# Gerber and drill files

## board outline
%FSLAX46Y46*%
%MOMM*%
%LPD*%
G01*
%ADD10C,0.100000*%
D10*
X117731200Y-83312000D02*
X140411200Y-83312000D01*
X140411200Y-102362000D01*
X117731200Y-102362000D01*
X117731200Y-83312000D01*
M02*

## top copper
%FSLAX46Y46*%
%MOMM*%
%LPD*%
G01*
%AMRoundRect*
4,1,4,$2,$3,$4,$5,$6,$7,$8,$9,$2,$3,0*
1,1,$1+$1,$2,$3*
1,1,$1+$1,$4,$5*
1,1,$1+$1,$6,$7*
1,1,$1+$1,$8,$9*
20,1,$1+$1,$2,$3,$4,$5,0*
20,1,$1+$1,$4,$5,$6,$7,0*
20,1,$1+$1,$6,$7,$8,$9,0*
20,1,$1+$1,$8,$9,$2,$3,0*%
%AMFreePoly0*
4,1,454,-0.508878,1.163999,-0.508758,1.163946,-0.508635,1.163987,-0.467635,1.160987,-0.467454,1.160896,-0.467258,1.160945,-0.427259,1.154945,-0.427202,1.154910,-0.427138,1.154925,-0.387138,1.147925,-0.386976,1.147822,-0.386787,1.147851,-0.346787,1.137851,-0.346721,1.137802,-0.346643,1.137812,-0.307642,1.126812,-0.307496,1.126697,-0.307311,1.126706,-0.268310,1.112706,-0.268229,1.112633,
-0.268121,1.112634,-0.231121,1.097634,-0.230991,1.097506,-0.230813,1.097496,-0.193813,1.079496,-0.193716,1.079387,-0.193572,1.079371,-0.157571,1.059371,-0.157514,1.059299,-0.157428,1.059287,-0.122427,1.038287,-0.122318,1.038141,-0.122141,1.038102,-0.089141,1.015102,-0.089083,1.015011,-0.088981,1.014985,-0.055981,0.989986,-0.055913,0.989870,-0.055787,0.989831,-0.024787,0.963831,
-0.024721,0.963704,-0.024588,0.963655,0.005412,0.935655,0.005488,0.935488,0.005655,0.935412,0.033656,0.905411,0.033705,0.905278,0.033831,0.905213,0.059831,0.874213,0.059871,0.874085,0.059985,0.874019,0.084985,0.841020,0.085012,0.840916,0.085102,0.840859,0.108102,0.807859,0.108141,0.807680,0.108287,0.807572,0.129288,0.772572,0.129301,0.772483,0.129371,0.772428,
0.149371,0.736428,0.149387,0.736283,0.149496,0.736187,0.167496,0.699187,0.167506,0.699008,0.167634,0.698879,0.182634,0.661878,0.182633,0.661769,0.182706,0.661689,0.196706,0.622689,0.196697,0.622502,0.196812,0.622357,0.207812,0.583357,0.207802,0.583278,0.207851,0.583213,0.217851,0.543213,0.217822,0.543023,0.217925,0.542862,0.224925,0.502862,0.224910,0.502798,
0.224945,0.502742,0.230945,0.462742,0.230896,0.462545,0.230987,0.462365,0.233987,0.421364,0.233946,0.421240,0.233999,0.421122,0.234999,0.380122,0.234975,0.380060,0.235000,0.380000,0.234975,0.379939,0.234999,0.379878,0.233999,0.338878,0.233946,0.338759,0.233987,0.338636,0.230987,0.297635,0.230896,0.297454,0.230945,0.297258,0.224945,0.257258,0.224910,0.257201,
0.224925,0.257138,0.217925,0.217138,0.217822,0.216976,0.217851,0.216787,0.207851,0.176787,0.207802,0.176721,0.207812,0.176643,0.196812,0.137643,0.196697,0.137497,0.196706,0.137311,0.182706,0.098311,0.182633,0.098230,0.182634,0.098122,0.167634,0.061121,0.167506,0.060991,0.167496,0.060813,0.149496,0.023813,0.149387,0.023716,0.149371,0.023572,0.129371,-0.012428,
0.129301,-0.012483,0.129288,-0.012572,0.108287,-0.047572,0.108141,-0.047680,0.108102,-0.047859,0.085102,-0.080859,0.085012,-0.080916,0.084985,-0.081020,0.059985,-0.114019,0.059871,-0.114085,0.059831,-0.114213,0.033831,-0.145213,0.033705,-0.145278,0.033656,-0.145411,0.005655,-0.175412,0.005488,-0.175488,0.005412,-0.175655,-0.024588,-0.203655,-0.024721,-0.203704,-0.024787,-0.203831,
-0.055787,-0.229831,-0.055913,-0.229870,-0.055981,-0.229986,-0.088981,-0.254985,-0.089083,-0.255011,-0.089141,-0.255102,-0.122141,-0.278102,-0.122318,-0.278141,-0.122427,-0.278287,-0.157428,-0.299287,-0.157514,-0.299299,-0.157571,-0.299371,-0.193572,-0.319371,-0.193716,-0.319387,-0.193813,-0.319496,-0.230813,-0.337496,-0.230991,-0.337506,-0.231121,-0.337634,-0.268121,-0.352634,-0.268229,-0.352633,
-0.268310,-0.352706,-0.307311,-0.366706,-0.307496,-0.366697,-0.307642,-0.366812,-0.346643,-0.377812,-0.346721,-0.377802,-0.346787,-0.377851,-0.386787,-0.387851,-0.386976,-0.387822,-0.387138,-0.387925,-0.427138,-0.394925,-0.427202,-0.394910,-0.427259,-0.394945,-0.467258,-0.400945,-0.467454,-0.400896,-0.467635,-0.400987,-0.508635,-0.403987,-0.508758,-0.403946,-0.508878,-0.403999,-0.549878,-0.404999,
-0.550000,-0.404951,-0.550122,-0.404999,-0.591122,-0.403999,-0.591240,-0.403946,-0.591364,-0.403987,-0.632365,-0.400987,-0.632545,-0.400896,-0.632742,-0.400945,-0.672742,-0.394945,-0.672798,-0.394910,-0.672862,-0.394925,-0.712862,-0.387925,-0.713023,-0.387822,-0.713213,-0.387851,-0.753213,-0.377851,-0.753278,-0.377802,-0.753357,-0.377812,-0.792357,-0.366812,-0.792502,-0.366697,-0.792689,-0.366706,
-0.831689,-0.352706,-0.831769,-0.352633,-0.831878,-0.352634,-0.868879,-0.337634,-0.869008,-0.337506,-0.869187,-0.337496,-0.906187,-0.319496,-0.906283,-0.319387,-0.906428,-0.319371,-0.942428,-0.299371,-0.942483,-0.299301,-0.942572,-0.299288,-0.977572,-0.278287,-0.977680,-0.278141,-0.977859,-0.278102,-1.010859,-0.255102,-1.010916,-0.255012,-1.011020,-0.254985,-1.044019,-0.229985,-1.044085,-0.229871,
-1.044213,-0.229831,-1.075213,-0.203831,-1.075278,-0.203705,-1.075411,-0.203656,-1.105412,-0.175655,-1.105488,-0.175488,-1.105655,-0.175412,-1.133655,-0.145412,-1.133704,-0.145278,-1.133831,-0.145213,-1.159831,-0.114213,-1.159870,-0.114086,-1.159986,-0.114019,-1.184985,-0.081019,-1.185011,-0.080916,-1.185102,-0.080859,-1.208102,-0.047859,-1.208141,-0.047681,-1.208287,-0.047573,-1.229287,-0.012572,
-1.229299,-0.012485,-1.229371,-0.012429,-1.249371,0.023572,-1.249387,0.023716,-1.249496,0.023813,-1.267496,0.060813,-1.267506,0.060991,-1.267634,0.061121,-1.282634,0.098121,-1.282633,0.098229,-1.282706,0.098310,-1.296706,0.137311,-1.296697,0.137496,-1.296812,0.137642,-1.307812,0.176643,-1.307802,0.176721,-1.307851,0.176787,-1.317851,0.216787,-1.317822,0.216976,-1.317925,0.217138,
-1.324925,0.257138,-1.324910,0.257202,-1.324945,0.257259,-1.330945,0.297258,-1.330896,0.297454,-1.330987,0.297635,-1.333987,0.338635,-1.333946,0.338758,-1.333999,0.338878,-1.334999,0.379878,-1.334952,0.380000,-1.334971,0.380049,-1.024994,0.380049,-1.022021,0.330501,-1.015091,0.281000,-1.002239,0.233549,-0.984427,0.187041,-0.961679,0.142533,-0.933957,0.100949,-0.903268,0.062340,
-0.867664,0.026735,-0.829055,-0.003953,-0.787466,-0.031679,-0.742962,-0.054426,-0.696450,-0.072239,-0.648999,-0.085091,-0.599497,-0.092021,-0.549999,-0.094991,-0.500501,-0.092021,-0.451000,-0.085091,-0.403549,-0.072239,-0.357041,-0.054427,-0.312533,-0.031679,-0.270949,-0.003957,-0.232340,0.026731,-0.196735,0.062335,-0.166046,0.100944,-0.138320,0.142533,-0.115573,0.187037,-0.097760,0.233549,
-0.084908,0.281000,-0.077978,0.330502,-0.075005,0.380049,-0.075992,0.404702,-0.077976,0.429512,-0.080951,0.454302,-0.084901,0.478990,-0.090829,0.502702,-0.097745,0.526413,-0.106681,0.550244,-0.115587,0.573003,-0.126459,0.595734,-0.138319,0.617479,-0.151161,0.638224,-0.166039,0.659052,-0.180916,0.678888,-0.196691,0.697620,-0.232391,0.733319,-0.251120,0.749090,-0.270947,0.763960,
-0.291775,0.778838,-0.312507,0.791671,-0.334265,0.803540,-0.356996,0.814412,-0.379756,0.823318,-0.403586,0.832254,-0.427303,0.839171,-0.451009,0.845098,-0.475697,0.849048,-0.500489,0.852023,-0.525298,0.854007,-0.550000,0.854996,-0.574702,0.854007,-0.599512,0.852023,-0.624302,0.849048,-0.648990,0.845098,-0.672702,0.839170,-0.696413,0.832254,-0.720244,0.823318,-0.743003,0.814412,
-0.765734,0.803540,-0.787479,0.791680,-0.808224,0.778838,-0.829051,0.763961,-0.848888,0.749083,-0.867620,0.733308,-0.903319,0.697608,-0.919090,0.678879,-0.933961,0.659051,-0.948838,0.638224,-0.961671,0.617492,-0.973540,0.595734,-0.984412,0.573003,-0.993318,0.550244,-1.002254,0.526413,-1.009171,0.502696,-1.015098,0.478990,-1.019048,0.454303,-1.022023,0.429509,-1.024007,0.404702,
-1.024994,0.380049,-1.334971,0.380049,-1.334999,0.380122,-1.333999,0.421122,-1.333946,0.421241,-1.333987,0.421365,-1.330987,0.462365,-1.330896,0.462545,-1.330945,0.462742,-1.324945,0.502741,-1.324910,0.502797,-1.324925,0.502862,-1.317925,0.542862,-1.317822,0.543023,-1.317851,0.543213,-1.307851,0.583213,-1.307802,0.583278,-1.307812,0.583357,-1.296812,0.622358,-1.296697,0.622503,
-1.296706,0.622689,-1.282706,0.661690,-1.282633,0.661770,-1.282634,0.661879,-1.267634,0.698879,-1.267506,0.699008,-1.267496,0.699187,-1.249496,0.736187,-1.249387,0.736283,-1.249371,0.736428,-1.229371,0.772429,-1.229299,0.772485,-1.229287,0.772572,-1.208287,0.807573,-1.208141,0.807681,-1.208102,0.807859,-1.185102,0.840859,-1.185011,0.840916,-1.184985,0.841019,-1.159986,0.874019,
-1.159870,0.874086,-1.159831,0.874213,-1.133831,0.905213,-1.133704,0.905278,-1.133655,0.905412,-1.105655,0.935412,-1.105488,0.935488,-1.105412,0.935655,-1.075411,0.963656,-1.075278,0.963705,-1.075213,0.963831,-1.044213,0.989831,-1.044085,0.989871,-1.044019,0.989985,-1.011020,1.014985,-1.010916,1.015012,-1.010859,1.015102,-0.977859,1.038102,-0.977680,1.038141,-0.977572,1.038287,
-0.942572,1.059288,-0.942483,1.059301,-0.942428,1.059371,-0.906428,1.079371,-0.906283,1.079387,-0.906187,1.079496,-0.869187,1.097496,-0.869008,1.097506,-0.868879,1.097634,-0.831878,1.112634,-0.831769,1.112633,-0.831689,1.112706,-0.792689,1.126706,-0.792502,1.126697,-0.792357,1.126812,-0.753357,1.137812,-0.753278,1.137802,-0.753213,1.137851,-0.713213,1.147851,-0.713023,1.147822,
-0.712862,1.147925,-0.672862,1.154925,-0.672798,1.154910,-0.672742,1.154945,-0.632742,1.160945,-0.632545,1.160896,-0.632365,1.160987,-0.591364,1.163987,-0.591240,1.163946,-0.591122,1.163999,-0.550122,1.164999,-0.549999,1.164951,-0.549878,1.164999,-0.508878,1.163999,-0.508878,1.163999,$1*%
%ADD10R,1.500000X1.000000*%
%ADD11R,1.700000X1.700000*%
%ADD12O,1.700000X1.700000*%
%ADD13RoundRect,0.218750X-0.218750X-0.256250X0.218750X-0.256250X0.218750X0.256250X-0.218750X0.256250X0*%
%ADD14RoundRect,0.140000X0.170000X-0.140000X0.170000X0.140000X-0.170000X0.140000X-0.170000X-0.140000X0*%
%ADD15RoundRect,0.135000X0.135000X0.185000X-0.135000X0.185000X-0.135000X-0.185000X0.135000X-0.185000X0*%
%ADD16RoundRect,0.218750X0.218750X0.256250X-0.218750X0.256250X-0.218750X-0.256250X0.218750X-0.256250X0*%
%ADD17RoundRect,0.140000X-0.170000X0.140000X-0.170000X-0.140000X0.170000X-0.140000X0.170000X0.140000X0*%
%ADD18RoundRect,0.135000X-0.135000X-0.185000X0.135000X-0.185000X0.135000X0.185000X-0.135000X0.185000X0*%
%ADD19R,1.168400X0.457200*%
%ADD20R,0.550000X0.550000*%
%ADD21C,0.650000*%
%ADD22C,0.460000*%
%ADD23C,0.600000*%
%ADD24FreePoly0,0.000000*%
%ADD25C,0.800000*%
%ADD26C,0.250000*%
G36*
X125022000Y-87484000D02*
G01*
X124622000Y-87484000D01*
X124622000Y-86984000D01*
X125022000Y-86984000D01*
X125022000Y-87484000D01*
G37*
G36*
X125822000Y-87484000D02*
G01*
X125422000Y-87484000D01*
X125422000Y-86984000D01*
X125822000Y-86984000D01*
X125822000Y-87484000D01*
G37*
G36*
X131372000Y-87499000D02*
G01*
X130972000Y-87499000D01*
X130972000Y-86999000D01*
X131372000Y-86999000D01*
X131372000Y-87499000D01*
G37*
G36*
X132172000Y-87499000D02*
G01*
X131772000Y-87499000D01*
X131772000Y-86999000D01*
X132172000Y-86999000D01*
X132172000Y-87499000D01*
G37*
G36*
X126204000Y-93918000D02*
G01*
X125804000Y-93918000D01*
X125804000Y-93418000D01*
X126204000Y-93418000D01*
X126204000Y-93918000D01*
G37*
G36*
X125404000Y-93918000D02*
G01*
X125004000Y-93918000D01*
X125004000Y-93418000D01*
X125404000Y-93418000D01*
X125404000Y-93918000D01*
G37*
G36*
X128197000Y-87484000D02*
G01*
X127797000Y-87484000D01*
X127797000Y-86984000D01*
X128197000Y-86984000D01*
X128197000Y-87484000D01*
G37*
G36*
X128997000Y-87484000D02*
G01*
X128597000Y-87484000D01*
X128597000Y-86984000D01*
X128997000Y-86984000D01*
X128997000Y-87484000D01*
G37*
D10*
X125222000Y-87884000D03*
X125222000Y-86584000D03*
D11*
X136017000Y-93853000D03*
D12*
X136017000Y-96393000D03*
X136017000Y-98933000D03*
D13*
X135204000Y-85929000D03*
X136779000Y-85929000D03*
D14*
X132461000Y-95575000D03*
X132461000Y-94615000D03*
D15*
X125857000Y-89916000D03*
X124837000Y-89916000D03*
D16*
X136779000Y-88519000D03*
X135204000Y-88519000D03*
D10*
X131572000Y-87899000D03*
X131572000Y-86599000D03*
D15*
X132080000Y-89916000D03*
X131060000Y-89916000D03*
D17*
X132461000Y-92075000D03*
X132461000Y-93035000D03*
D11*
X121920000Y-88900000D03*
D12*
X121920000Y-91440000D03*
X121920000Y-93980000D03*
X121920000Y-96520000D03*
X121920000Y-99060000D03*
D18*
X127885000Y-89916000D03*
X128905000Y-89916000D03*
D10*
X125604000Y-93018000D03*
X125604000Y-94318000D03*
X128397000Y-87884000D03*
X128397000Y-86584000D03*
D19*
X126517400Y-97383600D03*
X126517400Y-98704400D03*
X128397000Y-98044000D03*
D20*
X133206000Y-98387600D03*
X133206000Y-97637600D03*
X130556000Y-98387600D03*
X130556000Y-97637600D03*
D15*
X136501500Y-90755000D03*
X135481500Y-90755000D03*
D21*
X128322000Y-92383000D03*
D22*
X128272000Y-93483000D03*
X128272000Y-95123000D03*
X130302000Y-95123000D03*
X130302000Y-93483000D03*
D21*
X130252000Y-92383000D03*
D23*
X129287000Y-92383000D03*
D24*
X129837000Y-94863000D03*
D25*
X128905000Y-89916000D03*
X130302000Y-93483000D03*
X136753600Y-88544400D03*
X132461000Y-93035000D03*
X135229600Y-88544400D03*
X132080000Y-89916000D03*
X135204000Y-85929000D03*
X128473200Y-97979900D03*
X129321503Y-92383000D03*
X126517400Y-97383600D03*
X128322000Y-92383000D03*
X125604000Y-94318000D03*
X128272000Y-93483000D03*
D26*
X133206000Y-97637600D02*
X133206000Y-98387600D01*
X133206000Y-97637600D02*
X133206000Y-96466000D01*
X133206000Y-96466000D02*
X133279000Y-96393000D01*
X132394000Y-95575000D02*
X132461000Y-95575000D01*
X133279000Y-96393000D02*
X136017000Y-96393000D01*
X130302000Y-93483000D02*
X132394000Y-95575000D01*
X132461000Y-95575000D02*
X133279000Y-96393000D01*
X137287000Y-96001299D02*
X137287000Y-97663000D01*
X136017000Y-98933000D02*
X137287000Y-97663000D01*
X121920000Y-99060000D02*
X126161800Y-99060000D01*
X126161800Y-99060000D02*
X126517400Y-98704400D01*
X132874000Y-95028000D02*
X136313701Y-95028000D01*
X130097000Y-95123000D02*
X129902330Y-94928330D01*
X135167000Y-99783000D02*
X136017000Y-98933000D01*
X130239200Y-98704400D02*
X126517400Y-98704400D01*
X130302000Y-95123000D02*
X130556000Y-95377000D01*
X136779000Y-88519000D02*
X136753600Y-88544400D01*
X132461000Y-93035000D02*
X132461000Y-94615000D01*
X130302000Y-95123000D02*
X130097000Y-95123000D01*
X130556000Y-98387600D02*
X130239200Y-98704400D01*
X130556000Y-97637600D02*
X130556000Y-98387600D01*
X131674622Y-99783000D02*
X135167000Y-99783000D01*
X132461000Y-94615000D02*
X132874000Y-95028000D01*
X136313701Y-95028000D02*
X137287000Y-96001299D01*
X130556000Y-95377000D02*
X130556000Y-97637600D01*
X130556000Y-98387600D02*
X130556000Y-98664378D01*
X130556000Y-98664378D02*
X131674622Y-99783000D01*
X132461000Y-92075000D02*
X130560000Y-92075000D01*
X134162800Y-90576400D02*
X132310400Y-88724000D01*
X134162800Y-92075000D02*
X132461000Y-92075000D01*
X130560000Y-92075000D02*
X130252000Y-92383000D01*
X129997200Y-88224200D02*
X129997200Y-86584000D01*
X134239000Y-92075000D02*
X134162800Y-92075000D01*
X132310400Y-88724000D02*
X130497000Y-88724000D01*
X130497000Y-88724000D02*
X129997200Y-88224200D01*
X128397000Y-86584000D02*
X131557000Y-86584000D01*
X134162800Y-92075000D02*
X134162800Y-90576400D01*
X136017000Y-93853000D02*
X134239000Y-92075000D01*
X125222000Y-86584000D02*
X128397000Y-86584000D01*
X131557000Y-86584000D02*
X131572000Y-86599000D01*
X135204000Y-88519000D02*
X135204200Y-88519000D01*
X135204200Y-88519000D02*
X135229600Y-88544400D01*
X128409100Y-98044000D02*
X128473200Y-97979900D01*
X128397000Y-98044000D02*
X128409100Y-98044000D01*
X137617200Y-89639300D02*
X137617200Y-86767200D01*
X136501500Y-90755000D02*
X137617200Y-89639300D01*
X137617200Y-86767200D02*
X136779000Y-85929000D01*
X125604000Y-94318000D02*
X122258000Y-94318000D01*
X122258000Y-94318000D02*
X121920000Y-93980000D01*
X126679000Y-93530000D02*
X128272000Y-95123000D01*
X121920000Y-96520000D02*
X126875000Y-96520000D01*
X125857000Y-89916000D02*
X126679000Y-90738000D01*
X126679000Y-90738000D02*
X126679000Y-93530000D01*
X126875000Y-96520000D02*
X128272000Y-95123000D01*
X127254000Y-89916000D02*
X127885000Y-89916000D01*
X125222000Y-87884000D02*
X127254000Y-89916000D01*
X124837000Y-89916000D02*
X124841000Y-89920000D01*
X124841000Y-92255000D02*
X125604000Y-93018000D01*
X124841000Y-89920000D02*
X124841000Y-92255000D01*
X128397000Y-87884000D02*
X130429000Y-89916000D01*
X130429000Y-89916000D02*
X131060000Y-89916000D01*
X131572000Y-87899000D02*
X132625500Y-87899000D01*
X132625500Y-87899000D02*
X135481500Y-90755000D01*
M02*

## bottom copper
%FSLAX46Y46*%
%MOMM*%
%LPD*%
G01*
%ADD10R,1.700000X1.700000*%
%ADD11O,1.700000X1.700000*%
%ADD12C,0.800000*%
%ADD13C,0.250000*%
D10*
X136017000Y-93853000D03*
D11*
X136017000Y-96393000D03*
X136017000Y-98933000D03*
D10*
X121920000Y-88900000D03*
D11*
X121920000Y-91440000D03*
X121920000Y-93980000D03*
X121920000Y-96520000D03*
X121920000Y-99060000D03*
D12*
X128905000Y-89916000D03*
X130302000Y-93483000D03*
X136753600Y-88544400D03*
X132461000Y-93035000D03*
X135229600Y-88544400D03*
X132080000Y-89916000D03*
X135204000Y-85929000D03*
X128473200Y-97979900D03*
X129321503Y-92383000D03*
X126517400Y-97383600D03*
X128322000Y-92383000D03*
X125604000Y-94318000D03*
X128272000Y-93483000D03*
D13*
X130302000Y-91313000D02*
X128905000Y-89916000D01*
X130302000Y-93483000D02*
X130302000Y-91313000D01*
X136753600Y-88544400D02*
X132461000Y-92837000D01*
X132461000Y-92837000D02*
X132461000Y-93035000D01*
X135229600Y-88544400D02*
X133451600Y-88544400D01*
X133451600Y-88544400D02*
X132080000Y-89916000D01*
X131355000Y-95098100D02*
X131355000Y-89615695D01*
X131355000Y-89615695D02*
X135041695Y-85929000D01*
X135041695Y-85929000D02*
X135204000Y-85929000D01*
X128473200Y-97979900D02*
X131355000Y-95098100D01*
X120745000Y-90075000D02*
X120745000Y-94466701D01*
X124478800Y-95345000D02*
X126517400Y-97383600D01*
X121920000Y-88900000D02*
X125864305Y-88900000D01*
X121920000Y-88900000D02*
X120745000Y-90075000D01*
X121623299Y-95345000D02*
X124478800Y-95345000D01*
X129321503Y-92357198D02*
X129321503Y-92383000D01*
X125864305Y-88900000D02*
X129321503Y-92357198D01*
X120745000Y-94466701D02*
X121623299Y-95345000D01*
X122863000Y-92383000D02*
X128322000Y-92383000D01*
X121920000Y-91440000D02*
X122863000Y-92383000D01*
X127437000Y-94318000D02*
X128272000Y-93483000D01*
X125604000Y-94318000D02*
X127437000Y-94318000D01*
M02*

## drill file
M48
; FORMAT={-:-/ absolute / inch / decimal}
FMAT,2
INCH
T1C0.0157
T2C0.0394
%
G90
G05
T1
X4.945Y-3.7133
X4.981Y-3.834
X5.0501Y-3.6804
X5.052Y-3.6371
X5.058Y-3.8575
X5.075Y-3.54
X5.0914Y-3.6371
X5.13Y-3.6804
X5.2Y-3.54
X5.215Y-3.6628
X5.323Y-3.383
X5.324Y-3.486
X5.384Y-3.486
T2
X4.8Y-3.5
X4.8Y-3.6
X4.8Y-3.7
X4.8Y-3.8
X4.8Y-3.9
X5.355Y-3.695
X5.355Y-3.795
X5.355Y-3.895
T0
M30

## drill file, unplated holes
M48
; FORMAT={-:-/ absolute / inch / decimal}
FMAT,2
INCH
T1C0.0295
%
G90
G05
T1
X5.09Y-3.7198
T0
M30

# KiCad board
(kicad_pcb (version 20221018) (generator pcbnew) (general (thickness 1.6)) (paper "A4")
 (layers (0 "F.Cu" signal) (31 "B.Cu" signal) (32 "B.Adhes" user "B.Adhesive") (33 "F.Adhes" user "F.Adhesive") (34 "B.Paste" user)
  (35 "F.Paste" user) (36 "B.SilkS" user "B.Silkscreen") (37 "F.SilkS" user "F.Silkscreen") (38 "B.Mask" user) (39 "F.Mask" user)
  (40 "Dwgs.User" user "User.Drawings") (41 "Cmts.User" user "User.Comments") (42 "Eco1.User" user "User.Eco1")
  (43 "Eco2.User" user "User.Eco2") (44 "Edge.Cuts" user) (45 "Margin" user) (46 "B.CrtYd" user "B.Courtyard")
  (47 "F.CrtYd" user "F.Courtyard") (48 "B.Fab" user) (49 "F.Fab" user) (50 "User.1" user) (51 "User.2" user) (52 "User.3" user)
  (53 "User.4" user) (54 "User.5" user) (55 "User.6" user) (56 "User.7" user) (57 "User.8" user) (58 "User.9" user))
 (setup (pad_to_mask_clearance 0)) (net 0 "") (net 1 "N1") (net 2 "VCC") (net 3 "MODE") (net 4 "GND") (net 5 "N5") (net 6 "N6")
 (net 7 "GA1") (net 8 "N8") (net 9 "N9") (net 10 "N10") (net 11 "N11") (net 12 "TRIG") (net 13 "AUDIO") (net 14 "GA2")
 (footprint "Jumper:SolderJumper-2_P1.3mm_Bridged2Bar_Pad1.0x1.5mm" (layer "F.Cu") (at 125.222 87.234 90) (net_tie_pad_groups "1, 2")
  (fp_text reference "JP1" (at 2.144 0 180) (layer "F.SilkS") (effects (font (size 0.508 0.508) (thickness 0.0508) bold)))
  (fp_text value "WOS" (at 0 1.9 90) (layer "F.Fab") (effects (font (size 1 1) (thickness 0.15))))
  (fp_poly (pts (xy -0.25 -0.6) (xy 0.25 -0.6) (xy 0.25 -0.2) (xy -0.25 -0.2)) (stroke (width 0) (type solid)) (fill solid) (layer "F.Cu"))
  (fp_poly (pts (xy -0.25 0.2) (xy 0.25 0.2) (xy 0.25 0.6) (xy -0.25 0.6)) (stroke (width 0) (type solid)) (fill solid) (layer "F.Cu"))
  (pad "1" smd rect (at -0.65 0 90) (size 1 1.5) (layers "F.Cu" "F.Mask") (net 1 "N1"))
  (pad "2" smd rect (at 0.65 0 90) (size 1 1.5) (layers "F.Cu" "F.Mask") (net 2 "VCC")))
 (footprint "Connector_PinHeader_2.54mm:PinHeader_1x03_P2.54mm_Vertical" (layer "F.Cu") (at 136.017 93.853)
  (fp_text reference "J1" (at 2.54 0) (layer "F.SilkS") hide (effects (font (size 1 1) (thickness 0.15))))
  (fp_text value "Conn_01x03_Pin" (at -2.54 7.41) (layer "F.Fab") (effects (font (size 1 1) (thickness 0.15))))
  (pad "1" thru_hole rect (at 0 0) (size 1.7 1.7) (drill 1) (layers "*.Cu" "*.Mask" "F.SilkS") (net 2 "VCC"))
  (pad "2" thru_hole oval (at 0 2.54) (size 1.7 1.7) (drill 1) (layers "*.Cu" "*.Mask") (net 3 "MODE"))
  (pad "3" thru_hole oval (at 0 5.08) (size 1.7 1.7) (drill 1) (layers "*.Cu" "*.Mask") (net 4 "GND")))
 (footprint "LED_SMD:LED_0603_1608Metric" (layer "F.Cu") (at 135.9915 85.929)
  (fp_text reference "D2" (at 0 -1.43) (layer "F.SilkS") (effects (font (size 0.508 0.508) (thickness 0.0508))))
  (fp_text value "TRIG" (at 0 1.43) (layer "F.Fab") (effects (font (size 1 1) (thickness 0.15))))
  (pad "1" smd roundrect (at -0.7875 0) (size 0.875 0.95) (layers "F.Cu" "F.Paste" "F.Mask") (roundrect_rratio 0.25) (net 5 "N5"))
  (pad "2" smd roundrect (at 0.7875 0) (size 0.875 0.95) (layers "F.Cu" "F.Paste" "F.Mask") (roundrect_rratio 0.25) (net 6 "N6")))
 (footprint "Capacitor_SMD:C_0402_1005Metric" (layer "F.Cu") (at 132.461 95.095 90)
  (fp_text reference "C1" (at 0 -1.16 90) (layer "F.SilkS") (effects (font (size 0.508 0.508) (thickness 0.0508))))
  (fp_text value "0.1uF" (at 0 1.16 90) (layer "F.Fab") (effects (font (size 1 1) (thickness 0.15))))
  (pad "1" smd roundrect (at -0.48 0 90) (size 0.56 0.62) (layers "F.Cu" "F.Paste" "F.Mask") (roundrect_rratio 0.25) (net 3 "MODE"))
  (pad "2" smd roundrect (at 0.48 0 90) (size 0.56 0.62) (layers "F.Cu" "F.Paste" "F.Mask") (roundrect_rratio 0.25) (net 4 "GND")))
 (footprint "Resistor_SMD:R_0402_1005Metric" (layer "F.Cu") (at 125.347 89.916 180)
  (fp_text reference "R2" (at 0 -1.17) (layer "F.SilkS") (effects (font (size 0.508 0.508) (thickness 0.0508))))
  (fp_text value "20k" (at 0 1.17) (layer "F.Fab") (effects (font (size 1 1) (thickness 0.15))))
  (pad "1" smd roundrect (at -0.51 0 180) (size 0.54 0.64) (layers "F.Cu" "F.Paste" "F.Mask") (roundrect_rratio 0.25) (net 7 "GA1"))
  (pad "2" smd roundrect (at 0.51 0 180) (size 0.54 0.64) (layers "F.Cu" "F.Paste" "F.Mask") (roundrect_rratio 0.25) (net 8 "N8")))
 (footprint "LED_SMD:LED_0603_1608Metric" (layer "F.Cu") (at 135.9915 88.519 180)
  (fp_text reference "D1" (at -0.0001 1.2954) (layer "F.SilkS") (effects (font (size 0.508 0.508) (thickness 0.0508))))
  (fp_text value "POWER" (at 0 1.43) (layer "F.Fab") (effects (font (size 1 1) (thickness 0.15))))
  (pad "1" smd roundrect (at -0.7875 0 180) (size 0.875 0.95) (layers "F.Cu" "F.Paste" "F.Mask") (roundrect_rratio 0.25) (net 4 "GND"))
  (pad "2" smd roundrect (at 0.7875 0 180) (size 0.875 0.95) (layers "F.Cu" "F.Paste" "F.Mask") (roundrect_rratio 0.25) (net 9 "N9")))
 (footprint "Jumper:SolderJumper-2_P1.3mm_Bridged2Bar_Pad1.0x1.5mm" (layer "F.Cu") (at 131.572 87.249 90) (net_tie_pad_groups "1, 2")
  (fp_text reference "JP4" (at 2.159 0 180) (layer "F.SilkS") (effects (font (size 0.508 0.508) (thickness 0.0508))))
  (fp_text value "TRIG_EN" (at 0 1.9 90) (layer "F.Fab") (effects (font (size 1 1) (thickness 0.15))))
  (fp_poly (pts (xy -0.25 -0.6) (xy 0.25 -0.6) (xy 0.25 -0.2) (xy -0.25 -0.2)) (stroke (width 0) (type solid)) (fill solid) (layer "F.Cu"))
  (fp_poly (pts (xy -0.25 0.2) (xy 0.25 0.2) (xy 0.25 0.6) (xy -0.25 0.6)) (stroke (width 0) (type solid)) (fill solid) (layer "F.Cu"))
  (pad "1" smd rect (at -0.65 0 90) (size 1 1.5) (layers "F.Cu" "F.Mask") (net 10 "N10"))
  (pad "2" smd rect (at 0.65 0 90) (size 1 1.5) (layers "F.Cu" "F.Mask") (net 2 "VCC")))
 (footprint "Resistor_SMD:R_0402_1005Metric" (layer "F.Cu") (at 131.57 89.916 180)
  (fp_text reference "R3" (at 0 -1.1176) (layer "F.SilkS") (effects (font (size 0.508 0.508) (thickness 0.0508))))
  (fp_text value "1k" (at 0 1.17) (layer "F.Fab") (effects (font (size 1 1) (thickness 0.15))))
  (pad "1" smd roundrect (at -0.51 0 180) (size 0.54 0.64) (layers "F.Cu" "F.Paste" "F.Mask") (roundrect_rratio 0.25) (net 9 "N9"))
  (pad "2" smd roundrect (at 0.51 0 180) (size 0.54 0.64) (layers "F.Cu" "F.Paste" "F.Mask") (roundrect_rratio 0.25) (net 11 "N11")))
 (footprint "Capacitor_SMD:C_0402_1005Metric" (layer "F.Cu") (at 132.461 92.555 -90)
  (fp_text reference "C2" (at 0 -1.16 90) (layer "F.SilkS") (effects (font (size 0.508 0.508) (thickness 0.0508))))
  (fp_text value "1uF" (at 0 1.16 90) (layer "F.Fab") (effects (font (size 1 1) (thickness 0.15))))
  (pad "1" smd roundrect (at -0.48 0 270) (size 0.56 0.62) (layers "F.Cu" "F.Paste" "F.Mask") (roundrect_rratio 0.25) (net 2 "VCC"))
  (pad "2" smd roundrect (at 0.48 0 270) (size 0.56 0.62) (layers "F.Cu" "F.Paste" "F.Mask") (roundrect_rratio 0.25) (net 4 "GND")))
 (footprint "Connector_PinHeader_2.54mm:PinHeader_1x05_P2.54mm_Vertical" (layer "F.Cu") (at 121.92 88.9)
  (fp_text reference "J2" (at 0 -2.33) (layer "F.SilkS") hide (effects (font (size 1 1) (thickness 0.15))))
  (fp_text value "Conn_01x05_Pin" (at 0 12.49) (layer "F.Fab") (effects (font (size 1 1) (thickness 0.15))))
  (pad "1" thru_hole rect (at 0 0) (size 1.7 1.7) (drill 1) (layers "*.Cu" "*.Mask") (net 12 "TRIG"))
  (pad "2" thru_hole oval (at 0 2.54) (size 1.7 1.7) (drill 1) (layers "*.Cu" "*.Mask") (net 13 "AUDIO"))
  (pad "3" thru_hole oval (at 0 5.08) (size 1.7 1.7) (drill 1) (layers "*.Cu" "*.Mask") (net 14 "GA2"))
  (pad "4" thru_hole oval (at 0 7.62) (size 1.7 1.7) (drill 1) (layers "*.Cu" "*.Mask") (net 7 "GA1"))
  (pad "5" thru_hole oval (at 0 10.16) (size 1.7 1.7) (drill 1) (layers "*.Cu" "*.Mask") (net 4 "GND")))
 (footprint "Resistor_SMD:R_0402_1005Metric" (layer "F.Cu") (at 128.395 89.916)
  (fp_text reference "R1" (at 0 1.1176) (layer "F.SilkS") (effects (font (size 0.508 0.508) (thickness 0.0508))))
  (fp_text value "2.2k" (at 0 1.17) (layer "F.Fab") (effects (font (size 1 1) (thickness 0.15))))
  (pad "1" smd roundrect (at -0.51 0) (size 0.54 0.64) (layers "F.Cu" "F.Paste" "F.Mask") (roundrect_rratio 0.25) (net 1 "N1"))
  (pad "2" smd roundrect (at 0.51 0) (size 0.54 0.64) (layers "F.Cu" "F.Paste" "F.Mask") (roundrect_rratio 0.25) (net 3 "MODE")))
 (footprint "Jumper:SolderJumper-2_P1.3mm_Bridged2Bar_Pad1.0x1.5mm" (layer "F.Cu") (at 125.604 93.668 -90) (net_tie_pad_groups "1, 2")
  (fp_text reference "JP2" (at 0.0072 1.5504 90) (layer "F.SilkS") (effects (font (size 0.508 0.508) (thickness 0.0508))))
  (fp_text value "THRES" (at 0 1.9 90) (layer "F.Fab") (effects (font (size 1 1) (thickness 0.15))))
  (fp_poly (pts (xy -0.25 -0.6) (xy 0.25 -0.6) (xy 0.25 -0.2) (xy -0.25 -0.2)) (stroke (width 0) (type solid)) (fill solid) (layer "F.Cu"))
  (fp_poly (pts (xy -0.25 0.2) (xy 0.25 0.2) (xy 0.25 0.6) (xy -0.25 0.6)) (stroke (width 0) (type solid)) (fill solid) (layer "F.Cu"))
  (pad "1" smd rect (at -0.65 0 270) (size 1 1.5) (layers "F.Cu" "F.Mask") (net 8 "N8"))
  (pad "2" smd rect (at 0.65 0 270) (size 1 1.5) (layers "F.Cu" "F.Mask") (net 14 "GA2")))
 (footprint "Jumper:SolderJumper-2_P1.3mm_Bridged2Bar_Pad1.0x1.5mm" (layer "F.Cu") (at 128.397 87.234 90) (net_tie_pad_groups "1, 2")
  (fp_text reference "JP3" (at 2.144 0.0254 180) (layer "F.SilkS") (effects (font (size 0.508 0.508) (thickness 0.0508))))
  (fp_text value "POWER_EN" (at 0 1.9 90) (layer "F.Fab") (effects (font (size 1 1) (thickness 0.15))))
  (fp_poly (pts (xy -0.25 -0.6) (xy 0.25 -0.6) (xy 0.25 -0.2) (xy -0.25 -0.2)) (stroke (width 0) (type solid)) (fill solid) (layer "F.Cu"))
  (fp_poly (pts (xy -0.25 0.2) (xy 0.25 0.2) (xy 0.25 0.6) (xy -0.25 0.6)) (stroke (width 0) (type solid)) (fill solid) (layer "F.Cu"))
  (pad "1" smd rect (at -0.65 0 90) (size 1 1.5) (layers "F.Cu" "F.Mask") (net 11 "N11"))
  (pad "2" smd rect (at 0.65 0 90) (size 1 1.5) (layers "F.Cu" "F.Mask") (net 2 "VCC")))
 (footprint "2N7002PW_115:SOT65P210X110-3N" (layer "F.Cu") (at 127.4572 98.044)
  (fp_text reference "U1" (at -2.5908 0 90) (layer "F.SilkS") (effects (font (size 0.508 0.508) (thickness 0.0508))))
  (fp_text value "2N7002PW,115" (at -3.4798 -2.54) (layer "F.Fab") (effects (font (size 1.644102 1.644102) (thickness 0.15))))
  (pad "1" smd rect (at -0.9398 -0.6604) (size 1.1684 0.4572) (layers "F.Cu" "F.Paste" "F.Mask") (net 12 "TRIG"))
  (pad "2" smd rect (at -0.9398 0.6604) (size 1.1684 0.4572) (layers "F.Cu" "F.Paste" "F.Mask") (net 4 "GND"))
  (pad "3" smd rect (at 0.9398 0) (size 1.1684 0.4572) (layers "F.Cu" "F.Paste" "F.Mask") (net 5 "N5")))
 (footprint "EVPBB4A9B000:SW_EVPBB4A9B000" (layer "F.Cu") (at 131.881 98.0126 180)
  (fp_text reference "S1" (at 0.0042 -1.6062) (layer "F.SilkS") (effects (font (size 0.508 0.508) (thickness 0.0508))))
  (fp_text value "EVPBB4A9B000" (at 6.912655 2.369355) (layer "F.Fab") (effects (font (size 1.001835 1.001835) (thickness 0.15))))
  (pad "A1" smd rect (at -1.325 -0.375 180) (size 0.55 0.55) (layers "F.Cu" "F.Mask") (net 3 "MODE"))
  (pad "A2" smd rect (at -1.325 0.375 180) (size 0.55 0.55) (layers "F.Cu" "F.Mask") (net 3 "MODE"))
  (pad "B1" smd rect (at 1.325 -0.375 180) (size 0.55 0.55) (layers "F.Cu" "F.Mask") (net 4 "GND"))
  (pad "B2" smd rect (at 1.325 0.375 180) (size 0.55 0.55) (layers "F.Cu" "F.Mask") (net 4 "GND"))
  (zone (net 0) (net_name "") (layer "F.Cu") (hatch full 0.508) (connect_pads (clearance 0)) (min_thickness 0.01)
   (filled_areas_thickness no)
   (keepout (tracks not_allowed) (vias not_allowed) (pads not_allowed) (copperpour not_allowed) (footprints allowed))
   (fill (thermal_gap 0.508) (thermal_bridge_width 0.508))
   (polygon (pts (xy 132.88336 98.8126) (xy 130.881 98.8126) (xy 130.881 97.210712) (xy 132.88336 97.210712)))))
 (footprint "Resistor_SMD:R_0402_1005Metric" (layer "F.Cu") (at 135.9915 90.755 180)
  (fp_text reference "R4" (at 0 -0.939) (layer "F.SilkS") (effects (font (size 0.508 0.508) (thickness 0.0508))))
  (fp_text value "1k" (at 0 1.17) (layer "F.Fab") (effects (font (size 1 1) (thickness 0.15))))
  (pad "1" smd roundrect (at -0.51 0 180) (size 0.54 0.64) (layers "F.Cu" "F.Paste" "F.Mask") (roundrect_rratio 0.25) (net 6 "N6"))
  (pad "2" smd roundrect (at 0.51 0 180) (size 0.54 0.64) (layers "F.Cu" "F.Paste" "F.Mask") (roundrect_rratio 0.25) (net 10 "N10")))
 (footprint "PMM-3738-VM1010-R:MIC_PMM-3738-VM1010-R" (layer "F.Cu") (at 129.287 93.753)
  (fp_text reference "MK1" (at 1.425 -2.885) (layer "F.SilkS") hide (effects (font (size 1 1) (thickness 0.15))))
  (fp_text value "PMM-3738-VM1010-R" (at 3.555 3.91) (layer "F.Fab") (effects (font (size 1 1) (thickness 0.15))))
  (pad "" np_thru_hole circle (at 0 0.73) (size 0.75 0.75) (drill 0.75) (layers "*.Cu" "*.Mask"))
  (pad "1" smd circle (at -0.965 -1.37) (size 0.65 0.65) (layers "F.Cu" "F.Mask") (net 13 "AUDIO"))
  (pad "2" smd circle (at -1.015 -0.27) (size 0.46 0.46) (layers "F.Cu" "F.Mask") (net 14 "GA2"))
  (pad "3" smd circle (at -1.015 1.37) (size 0.46 0.46) (layers "F.Cu" "F.Mask") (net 7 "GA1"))
  (pad "4" smd circle (at 1.015 1.37) (size 0.46 0.46) (layers "F.Cu" "F.Mask") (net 4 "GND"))
  (pad "5" smd circle (at 1.015 -0.27) (size 0.46 0.46) (layers "F.Cu" "F.Mask") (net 3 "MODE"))
  (pad "6" smd circle (at 0.965 -1.37) (size 0.65 0.65) (layers "F.Cu" "F.Mask") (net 2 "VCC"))
  (pad "7" smd circle (at 0 -1.37) (size 0.6 0.6) (layers "F.Cu" "F.Mask") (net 12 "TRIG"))
  (pad "8" smd custom (at 0.55 1.11) (size 0.08 0.08) (layers "F.Cu" "F.Paste" "F.Mask") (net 4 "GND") (zone_connect 0)
   (thermal_bridge_angle 45) (options (clearance outline) (anchor rect)) (primitives)))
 (gr_rect (start 117.7312 83.312) (end 140.4112 102.362) (stroke (width 0.1) (type default)) (fill none) (layer "Edge.Cuts"))
 (segment (start 133.206 97.6376) (end 133.206 98.3876) (width 0.25) (layer "F.Cu") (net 3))
 (segment (start 133.206 97.6376) (end 133.206 96.466) (width 0.25) (layer "F.Cu") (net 3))
 (segment (start 133.206 96.466) (end 133.279 96.393) (width 0.25) (layer "F.Cu") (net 3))
 (segment (start 132.394 95.575) (end 132.461 95.575) (width 0.25) (layer "F.Cu") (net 3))
 (segment (start 133.279 96.393) (end 136.017 96.393) (width 0.25) (layer "F.Cu") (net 3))
 (segment (start 130.302 93.483) (end 132.394 95.575) (width 0.25) (layer "F.Cu") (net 3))
 (segment (start 132.461 95.575) (end 133.279 96.393) (width 0.25) (layer "F.Cu") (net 3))
 (via (at 128.905 89.916) (size 0.8) (drill 0.4) (layers "F.Cu" "B.Cu") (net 3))
 (via (at 130.302 93.483) (size 0.8) (drill 0.4) (layers "F.Cu" "B.Cu") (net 3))
 (segment (start 130.302 91.313) (end 128.905 89.916) (width 0.25) (layer "B.Cu") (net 3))
 (segment (start 130.302 93.483) (end 130.302 91.313) (width 0.25) (layer "B.Cu") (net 3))
 (segment (start 137.287 96.001299) (end 137.287 97.663) (width 0.25) (layer "F.Cu") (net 4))
 (segment (start 136.017 98.933) (end 137.287 97.663) (width 0.25) (layer "F.Cu") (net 4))
 (segment (start 121.92 99.06) (end 126.1618 99.06) (width 0.25) (layer "F.Cu") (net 4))
 (segment (start 126.1618 99.06) (end 126.5174 98.7044) (width 0.25) (layer "F.Cu") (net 4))
 (segment (start 132.874 95.028) (end 136.313701 95.028) (width 0.25) (layer "F.Cu") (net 4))
 (segment (start 130.097 95.123) (end 129.90233 94.92833) (width 0.25) (layer "F.Cu") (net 4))
 (segment (start 135.167 99.783) (end 136.017 98.933) (width 0.25) (layer "F.Cu") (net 4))
 (segment (start 130.2392 98.7044) (end 126.5174 98.7044) (width 0.25) (layer "F.Cu") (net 4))
 (segment (start 130.302 95.123) (end 130.556 95.377) (width 0.25) (layer "F.Cu") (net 4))
 (segment (start 136.779 88.519) (end 136.7536 88.5444) (width 0.25) (layer "F.Cu") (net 4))
 (segment (start 132.461 93.035) (end 132.461 94.615) (width 0.25) (layer "F.Cu") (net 4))
 (segment (start 130.302 95.123) (end 130.097 95.123) (width 0.25) (layer "F.Cu") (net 4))
 (segment (start 130.556 98.3876) (end 130.2392 98.7044) (width 0.25) (layer "F.Cu") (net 4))
 (segment (start 130.556 97.6376) (end 130.556 98.3876) (width 0.25) (layer "F.Cu") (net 4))
 (segment (start 131.674622 99.783) (end 135.167 99.783) (width 0.25) (layer "F.Cu") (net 4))
 (segment (start 132.461 94.615) (end 132.874 95.028) (width 0.25) (layer "F.Cu") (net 4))
 (segment (start 136.313701 95.028) (end 137.287 96.001299) (width 0.25) (layer "F.Cu") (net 4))
 (segment (start 130.556 95.377) (end 130.556 97.6376) (width 0.25) (layer "F.Cu") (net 4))
 (segment (start 130.556 98.3876) (end 130.556 98.664378) (width 0.25) (layer "F.Cu") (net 4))
 (segment (start 130.556 98.664378) (end 131.674622 99.783) (width 0.25) (layer "F.Cu") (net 4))
 (via (at 136.7536 88.5444) (size 0.8) (drill 0.4) (layers "F.Cu" "B.Cu") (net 4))
 (via (at 132.461 93.035) (size 0.8) (drill 0.4) (layers "F.Cu" "B.Cu") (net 4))
 (segment (start 136.7536 88.5444) (end 132.461 92.837) (width 0.25) (layer "B.Cu") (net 4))
 (segment (start 132.461 92.837) (end 132.461 93.035) (width 0.25) (layer "B.Cu") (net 4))
 (segment (start 132.461 92.075) (end 130.56 92.075) (width 0.25) (layer "F.Cu") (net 2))
 (segment (start 134.1628 90.5764) (end 132.3104 88.724) (width 0.25) (layer "F.Cu") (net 2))
 (segment (start 134.1628 92.075) (end 132.461 92.075) (width 0.25) (layer "F.Cu") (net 2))
 (segment (start 130.56 92.075) (end 130.252 92.383) (width 0.25) (layer "F.Cu") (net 2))
 (segment (start 129.9972 88.2242) (end 129.9972 86.584) (width 0.25) (layer "F.Cu") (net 2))
 (segment (start 134.239 92.075) (end 134.1628 92.075) (width 0.25) (layer "F.Cu") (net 2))
 (segment (start 132.3104 88.724) (end 130.497 88.724) (width 0.25) (layer "F.Cu") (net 2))
 (segment (start 130.497 88.724) (end 129.9972 88.2242) (width 0.25) (layer "F.Cu") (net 2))
 (segment (start 128.397 86.584) (end 131.557 86.584) (width 0.25) (layer "F.Cu") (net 2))
 (segment (start 134.1628 92.075) (end 134.1628 90.5764) (width 0.25) (layer "F.Cu") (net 2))
 (segment (start 136.017 93.853) (end 134.239 92.075) (width 0.25) (layer "F.Cu") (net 2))
 (segment (start 125.222 86.584) (end 128.397 86.584) (width 0.25) (layer "F.Cu") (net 2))
 (segment (start 131.557 86.584) (end 131.572 86.599) (width 0.25) (layer "F.Cu") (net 2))
 (segment (start 135.204 88.519) (end 135.2042 88.519) (width 0.25) (layer "F.Cu") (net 9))
 (segment (start 135.2042 88.519) (end 135.2296 88.5444) (width 0.25) (layer "F.Cu") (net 9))
 (via (at 135.2296 88.5444) (size 0.8) (drill 0.4) (layers "F.Cu" "B.Cu") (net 9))
 (via (at 132.08 89.916) (size 0.8) (drill 0.4) (layers "F.Cu" "B.Cu") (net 9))
 (segment (start 135.2296 88.5444) (end 133.4516 88.5444) (width 0.25) (layer "B.Cu") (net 9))
 (segment (start 133.4516 88.5444) (end 132.08 89.916) (width 0.25) (layer "B.Cu") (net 9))
 (segment (start 128.4091 98.044) (end 128.4732 97.9799) (width 0.25) (layer "F.Cu") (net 5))
 (segment (start 128.397 98.044) (end 128.4091 98.044) (width 0.25) (layer "F.Cu") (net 5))
 (via (at 135.204 85.929) (size 0.8) (drill 0.4) (layers "F.Cu" "B.Cu") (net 5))
 (via (at 128.4732 97.9799) (size 0.8) (drill 0.4) (layers "F.Cu" "B.Cu") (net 5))
 (segment (start 131.355 95.0981) (end 131.355 89.615695) (width 0.25) (layer "B.Cu") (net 5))
 (segment (start 131.355 89.615695) (end 135.041695 85.929) (width 0.25) (layer "B.Cu") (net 5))
 (segment (start 135.041695 85.929) (end 135.204 85.929) (width 0.25) (layer "B.Cu") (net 5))
 (segment (start 128.4732 97.9799) (end 131.355 95.0981) (width 0.25) (layer "B.Cu") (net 5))
 (segment (start 137.6172 89.6393) (end 137.6172 86.7672) (width 0.25) (layer "F.Cu") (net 6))
 (segment (start 136.5015 90.755) (end 137.6172 89.6393) (width 0.25) (layer "F.Cu") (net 6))
 (segment (start 137.6172 86.7672) (end 136.779 85.929) (width 0.25) (layer "F.Cu") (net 6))
 (via (at 129.321503 92.383) (size 0.8) (drill 0.4) (layers "F.Cu" "B.Cu") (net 12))
 (via (at 126.5174 97.3836) (size 0.8) (drill 0.4) (layers "F.Cu" "B.Cu") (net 12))
 (segment (start 120.745 90.075) (end 120.745 94.466701) (width 0.25) (layer "B.Cu") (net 12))
 (segment (start 124.4788 95.345) (end 126.5174 97.3836) (width 0.25) (layer "B.Cu") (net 12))
 (segment (start 121.92 88.9) (end 125.864305 88.9) (width 0.25) (layer "B.Cu") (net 12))
 (segment (start 121.92 88.9) (end 120.745 90.075) (width 0.25) (layer "B.Cu") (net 12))
 (segment (start 121.623299 95.345) (end 124.4788 95.345) (width 0.25) (layer "B.Cu") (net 12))
 (segment (start 129.321503 92.357198) (end 129.321503 92.383) (width 0.25) (layer "B.Cu") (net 12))
 (segment (start 125.864305 88.9) (end 129.321503 92.357198) (width 0.25) (layer "B.Cu") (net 12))
 (segment (start 120.745 94.466701) (end 121.623299 95.345) (width 0.25) (layer "B.Cu") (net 12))
 (via (at 128.322 92.383) (size 0.8) (drill 0.4) (layers "F.Cu" "B.Cu") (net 13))
 (segment (start 122.863 92.383) (end 128.322 92.383) (width 0.25) (layer "B.Cu") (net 13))
 (segment (start 121.92 91.44) (end 122.863 92.383) (width 0.25) (layer "B.Cu") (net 13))
 (segment (start 125.604 94.318) (end 122.258 94.318) (width 0.25) (layer "F.Cu") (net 14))
 (segment (start 122.258 94.318) (end 121.92 93.98) (width 0.25) (layer "F.Cu") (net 14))
 (via (at 125.604 94.318) (size 0.8) (drill 0.4) (layers "F.Cu" "B.Cu") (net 14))
 (via (at 128.272 93.483) (size 0.8) (drill 0.4) (layers "F.Cu" "B.Cu") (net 14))
 (segment (start 127.437 94.318) (end 128.272 93.483) (width 0.25) (layer "B.Cu") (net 14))
 (segment (start 125.604 94.318) (end 127.437 94.318) (width 0.25) (layer "B.Cu") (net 14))
 (segment (start 126.679 93.53) (end 128.272 95.123) (width 0.25) (layer "F.Cu") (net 7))
 (segment (start 121.92 96.52) (end 126.875 96.52) (width 0.25) (layer "F.Cu") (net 7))
 (segment (start 125.857 89.916) (end 126.679 90.738) (width 0.25) (layer "F.Cu") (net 7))
 (segment (start 126.679 90.738) (end 126.679 93.53) (width 0.25) (layer "F.Cu") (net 7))
 (segment (start 126.875 96.52) (end 128.272 95.123) (width 0.25) (layer "F.Cu") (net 7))
 (segment (start 127.254 89.916) (end 127.885 89.916) (width 0.25) (layer "F.Cu") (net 1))
 (segment (start 125.222 87.884) (end 127.254 89.916) (width 0.25) (layer "F.Cu") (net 1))
 (segment (start 124.837 89.916) (end 124.841 89.92) (width 0.25) (layer "F.Cu") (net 8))
 (segment (start 124.841 92.255) (end 125.604 93.018) (width 0.25) (layer "F.Cu") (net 8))
 (segment (start 124.841 89.92) (end 124.841 92.255) (width 0.25) (layer "F.Cu") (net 8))
 (segment (start 128.397 87.884) (end 130.429 89.916) (width 0.25) (layer "F.Cu") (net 11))
 (segment (start 130.429 89.916) (end 131.06 89.916) (width 0.25) (layer "F.Cu") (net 11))
 (segment (start 131.572 87.899) (end 132.6255 87.899) (width 0.25) (layer "F.Cu") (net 10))
 (segment (start 132.6255 87.899) (end 135.4815 90.755) (width 0.25) (layer "F.Cu") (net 10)))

